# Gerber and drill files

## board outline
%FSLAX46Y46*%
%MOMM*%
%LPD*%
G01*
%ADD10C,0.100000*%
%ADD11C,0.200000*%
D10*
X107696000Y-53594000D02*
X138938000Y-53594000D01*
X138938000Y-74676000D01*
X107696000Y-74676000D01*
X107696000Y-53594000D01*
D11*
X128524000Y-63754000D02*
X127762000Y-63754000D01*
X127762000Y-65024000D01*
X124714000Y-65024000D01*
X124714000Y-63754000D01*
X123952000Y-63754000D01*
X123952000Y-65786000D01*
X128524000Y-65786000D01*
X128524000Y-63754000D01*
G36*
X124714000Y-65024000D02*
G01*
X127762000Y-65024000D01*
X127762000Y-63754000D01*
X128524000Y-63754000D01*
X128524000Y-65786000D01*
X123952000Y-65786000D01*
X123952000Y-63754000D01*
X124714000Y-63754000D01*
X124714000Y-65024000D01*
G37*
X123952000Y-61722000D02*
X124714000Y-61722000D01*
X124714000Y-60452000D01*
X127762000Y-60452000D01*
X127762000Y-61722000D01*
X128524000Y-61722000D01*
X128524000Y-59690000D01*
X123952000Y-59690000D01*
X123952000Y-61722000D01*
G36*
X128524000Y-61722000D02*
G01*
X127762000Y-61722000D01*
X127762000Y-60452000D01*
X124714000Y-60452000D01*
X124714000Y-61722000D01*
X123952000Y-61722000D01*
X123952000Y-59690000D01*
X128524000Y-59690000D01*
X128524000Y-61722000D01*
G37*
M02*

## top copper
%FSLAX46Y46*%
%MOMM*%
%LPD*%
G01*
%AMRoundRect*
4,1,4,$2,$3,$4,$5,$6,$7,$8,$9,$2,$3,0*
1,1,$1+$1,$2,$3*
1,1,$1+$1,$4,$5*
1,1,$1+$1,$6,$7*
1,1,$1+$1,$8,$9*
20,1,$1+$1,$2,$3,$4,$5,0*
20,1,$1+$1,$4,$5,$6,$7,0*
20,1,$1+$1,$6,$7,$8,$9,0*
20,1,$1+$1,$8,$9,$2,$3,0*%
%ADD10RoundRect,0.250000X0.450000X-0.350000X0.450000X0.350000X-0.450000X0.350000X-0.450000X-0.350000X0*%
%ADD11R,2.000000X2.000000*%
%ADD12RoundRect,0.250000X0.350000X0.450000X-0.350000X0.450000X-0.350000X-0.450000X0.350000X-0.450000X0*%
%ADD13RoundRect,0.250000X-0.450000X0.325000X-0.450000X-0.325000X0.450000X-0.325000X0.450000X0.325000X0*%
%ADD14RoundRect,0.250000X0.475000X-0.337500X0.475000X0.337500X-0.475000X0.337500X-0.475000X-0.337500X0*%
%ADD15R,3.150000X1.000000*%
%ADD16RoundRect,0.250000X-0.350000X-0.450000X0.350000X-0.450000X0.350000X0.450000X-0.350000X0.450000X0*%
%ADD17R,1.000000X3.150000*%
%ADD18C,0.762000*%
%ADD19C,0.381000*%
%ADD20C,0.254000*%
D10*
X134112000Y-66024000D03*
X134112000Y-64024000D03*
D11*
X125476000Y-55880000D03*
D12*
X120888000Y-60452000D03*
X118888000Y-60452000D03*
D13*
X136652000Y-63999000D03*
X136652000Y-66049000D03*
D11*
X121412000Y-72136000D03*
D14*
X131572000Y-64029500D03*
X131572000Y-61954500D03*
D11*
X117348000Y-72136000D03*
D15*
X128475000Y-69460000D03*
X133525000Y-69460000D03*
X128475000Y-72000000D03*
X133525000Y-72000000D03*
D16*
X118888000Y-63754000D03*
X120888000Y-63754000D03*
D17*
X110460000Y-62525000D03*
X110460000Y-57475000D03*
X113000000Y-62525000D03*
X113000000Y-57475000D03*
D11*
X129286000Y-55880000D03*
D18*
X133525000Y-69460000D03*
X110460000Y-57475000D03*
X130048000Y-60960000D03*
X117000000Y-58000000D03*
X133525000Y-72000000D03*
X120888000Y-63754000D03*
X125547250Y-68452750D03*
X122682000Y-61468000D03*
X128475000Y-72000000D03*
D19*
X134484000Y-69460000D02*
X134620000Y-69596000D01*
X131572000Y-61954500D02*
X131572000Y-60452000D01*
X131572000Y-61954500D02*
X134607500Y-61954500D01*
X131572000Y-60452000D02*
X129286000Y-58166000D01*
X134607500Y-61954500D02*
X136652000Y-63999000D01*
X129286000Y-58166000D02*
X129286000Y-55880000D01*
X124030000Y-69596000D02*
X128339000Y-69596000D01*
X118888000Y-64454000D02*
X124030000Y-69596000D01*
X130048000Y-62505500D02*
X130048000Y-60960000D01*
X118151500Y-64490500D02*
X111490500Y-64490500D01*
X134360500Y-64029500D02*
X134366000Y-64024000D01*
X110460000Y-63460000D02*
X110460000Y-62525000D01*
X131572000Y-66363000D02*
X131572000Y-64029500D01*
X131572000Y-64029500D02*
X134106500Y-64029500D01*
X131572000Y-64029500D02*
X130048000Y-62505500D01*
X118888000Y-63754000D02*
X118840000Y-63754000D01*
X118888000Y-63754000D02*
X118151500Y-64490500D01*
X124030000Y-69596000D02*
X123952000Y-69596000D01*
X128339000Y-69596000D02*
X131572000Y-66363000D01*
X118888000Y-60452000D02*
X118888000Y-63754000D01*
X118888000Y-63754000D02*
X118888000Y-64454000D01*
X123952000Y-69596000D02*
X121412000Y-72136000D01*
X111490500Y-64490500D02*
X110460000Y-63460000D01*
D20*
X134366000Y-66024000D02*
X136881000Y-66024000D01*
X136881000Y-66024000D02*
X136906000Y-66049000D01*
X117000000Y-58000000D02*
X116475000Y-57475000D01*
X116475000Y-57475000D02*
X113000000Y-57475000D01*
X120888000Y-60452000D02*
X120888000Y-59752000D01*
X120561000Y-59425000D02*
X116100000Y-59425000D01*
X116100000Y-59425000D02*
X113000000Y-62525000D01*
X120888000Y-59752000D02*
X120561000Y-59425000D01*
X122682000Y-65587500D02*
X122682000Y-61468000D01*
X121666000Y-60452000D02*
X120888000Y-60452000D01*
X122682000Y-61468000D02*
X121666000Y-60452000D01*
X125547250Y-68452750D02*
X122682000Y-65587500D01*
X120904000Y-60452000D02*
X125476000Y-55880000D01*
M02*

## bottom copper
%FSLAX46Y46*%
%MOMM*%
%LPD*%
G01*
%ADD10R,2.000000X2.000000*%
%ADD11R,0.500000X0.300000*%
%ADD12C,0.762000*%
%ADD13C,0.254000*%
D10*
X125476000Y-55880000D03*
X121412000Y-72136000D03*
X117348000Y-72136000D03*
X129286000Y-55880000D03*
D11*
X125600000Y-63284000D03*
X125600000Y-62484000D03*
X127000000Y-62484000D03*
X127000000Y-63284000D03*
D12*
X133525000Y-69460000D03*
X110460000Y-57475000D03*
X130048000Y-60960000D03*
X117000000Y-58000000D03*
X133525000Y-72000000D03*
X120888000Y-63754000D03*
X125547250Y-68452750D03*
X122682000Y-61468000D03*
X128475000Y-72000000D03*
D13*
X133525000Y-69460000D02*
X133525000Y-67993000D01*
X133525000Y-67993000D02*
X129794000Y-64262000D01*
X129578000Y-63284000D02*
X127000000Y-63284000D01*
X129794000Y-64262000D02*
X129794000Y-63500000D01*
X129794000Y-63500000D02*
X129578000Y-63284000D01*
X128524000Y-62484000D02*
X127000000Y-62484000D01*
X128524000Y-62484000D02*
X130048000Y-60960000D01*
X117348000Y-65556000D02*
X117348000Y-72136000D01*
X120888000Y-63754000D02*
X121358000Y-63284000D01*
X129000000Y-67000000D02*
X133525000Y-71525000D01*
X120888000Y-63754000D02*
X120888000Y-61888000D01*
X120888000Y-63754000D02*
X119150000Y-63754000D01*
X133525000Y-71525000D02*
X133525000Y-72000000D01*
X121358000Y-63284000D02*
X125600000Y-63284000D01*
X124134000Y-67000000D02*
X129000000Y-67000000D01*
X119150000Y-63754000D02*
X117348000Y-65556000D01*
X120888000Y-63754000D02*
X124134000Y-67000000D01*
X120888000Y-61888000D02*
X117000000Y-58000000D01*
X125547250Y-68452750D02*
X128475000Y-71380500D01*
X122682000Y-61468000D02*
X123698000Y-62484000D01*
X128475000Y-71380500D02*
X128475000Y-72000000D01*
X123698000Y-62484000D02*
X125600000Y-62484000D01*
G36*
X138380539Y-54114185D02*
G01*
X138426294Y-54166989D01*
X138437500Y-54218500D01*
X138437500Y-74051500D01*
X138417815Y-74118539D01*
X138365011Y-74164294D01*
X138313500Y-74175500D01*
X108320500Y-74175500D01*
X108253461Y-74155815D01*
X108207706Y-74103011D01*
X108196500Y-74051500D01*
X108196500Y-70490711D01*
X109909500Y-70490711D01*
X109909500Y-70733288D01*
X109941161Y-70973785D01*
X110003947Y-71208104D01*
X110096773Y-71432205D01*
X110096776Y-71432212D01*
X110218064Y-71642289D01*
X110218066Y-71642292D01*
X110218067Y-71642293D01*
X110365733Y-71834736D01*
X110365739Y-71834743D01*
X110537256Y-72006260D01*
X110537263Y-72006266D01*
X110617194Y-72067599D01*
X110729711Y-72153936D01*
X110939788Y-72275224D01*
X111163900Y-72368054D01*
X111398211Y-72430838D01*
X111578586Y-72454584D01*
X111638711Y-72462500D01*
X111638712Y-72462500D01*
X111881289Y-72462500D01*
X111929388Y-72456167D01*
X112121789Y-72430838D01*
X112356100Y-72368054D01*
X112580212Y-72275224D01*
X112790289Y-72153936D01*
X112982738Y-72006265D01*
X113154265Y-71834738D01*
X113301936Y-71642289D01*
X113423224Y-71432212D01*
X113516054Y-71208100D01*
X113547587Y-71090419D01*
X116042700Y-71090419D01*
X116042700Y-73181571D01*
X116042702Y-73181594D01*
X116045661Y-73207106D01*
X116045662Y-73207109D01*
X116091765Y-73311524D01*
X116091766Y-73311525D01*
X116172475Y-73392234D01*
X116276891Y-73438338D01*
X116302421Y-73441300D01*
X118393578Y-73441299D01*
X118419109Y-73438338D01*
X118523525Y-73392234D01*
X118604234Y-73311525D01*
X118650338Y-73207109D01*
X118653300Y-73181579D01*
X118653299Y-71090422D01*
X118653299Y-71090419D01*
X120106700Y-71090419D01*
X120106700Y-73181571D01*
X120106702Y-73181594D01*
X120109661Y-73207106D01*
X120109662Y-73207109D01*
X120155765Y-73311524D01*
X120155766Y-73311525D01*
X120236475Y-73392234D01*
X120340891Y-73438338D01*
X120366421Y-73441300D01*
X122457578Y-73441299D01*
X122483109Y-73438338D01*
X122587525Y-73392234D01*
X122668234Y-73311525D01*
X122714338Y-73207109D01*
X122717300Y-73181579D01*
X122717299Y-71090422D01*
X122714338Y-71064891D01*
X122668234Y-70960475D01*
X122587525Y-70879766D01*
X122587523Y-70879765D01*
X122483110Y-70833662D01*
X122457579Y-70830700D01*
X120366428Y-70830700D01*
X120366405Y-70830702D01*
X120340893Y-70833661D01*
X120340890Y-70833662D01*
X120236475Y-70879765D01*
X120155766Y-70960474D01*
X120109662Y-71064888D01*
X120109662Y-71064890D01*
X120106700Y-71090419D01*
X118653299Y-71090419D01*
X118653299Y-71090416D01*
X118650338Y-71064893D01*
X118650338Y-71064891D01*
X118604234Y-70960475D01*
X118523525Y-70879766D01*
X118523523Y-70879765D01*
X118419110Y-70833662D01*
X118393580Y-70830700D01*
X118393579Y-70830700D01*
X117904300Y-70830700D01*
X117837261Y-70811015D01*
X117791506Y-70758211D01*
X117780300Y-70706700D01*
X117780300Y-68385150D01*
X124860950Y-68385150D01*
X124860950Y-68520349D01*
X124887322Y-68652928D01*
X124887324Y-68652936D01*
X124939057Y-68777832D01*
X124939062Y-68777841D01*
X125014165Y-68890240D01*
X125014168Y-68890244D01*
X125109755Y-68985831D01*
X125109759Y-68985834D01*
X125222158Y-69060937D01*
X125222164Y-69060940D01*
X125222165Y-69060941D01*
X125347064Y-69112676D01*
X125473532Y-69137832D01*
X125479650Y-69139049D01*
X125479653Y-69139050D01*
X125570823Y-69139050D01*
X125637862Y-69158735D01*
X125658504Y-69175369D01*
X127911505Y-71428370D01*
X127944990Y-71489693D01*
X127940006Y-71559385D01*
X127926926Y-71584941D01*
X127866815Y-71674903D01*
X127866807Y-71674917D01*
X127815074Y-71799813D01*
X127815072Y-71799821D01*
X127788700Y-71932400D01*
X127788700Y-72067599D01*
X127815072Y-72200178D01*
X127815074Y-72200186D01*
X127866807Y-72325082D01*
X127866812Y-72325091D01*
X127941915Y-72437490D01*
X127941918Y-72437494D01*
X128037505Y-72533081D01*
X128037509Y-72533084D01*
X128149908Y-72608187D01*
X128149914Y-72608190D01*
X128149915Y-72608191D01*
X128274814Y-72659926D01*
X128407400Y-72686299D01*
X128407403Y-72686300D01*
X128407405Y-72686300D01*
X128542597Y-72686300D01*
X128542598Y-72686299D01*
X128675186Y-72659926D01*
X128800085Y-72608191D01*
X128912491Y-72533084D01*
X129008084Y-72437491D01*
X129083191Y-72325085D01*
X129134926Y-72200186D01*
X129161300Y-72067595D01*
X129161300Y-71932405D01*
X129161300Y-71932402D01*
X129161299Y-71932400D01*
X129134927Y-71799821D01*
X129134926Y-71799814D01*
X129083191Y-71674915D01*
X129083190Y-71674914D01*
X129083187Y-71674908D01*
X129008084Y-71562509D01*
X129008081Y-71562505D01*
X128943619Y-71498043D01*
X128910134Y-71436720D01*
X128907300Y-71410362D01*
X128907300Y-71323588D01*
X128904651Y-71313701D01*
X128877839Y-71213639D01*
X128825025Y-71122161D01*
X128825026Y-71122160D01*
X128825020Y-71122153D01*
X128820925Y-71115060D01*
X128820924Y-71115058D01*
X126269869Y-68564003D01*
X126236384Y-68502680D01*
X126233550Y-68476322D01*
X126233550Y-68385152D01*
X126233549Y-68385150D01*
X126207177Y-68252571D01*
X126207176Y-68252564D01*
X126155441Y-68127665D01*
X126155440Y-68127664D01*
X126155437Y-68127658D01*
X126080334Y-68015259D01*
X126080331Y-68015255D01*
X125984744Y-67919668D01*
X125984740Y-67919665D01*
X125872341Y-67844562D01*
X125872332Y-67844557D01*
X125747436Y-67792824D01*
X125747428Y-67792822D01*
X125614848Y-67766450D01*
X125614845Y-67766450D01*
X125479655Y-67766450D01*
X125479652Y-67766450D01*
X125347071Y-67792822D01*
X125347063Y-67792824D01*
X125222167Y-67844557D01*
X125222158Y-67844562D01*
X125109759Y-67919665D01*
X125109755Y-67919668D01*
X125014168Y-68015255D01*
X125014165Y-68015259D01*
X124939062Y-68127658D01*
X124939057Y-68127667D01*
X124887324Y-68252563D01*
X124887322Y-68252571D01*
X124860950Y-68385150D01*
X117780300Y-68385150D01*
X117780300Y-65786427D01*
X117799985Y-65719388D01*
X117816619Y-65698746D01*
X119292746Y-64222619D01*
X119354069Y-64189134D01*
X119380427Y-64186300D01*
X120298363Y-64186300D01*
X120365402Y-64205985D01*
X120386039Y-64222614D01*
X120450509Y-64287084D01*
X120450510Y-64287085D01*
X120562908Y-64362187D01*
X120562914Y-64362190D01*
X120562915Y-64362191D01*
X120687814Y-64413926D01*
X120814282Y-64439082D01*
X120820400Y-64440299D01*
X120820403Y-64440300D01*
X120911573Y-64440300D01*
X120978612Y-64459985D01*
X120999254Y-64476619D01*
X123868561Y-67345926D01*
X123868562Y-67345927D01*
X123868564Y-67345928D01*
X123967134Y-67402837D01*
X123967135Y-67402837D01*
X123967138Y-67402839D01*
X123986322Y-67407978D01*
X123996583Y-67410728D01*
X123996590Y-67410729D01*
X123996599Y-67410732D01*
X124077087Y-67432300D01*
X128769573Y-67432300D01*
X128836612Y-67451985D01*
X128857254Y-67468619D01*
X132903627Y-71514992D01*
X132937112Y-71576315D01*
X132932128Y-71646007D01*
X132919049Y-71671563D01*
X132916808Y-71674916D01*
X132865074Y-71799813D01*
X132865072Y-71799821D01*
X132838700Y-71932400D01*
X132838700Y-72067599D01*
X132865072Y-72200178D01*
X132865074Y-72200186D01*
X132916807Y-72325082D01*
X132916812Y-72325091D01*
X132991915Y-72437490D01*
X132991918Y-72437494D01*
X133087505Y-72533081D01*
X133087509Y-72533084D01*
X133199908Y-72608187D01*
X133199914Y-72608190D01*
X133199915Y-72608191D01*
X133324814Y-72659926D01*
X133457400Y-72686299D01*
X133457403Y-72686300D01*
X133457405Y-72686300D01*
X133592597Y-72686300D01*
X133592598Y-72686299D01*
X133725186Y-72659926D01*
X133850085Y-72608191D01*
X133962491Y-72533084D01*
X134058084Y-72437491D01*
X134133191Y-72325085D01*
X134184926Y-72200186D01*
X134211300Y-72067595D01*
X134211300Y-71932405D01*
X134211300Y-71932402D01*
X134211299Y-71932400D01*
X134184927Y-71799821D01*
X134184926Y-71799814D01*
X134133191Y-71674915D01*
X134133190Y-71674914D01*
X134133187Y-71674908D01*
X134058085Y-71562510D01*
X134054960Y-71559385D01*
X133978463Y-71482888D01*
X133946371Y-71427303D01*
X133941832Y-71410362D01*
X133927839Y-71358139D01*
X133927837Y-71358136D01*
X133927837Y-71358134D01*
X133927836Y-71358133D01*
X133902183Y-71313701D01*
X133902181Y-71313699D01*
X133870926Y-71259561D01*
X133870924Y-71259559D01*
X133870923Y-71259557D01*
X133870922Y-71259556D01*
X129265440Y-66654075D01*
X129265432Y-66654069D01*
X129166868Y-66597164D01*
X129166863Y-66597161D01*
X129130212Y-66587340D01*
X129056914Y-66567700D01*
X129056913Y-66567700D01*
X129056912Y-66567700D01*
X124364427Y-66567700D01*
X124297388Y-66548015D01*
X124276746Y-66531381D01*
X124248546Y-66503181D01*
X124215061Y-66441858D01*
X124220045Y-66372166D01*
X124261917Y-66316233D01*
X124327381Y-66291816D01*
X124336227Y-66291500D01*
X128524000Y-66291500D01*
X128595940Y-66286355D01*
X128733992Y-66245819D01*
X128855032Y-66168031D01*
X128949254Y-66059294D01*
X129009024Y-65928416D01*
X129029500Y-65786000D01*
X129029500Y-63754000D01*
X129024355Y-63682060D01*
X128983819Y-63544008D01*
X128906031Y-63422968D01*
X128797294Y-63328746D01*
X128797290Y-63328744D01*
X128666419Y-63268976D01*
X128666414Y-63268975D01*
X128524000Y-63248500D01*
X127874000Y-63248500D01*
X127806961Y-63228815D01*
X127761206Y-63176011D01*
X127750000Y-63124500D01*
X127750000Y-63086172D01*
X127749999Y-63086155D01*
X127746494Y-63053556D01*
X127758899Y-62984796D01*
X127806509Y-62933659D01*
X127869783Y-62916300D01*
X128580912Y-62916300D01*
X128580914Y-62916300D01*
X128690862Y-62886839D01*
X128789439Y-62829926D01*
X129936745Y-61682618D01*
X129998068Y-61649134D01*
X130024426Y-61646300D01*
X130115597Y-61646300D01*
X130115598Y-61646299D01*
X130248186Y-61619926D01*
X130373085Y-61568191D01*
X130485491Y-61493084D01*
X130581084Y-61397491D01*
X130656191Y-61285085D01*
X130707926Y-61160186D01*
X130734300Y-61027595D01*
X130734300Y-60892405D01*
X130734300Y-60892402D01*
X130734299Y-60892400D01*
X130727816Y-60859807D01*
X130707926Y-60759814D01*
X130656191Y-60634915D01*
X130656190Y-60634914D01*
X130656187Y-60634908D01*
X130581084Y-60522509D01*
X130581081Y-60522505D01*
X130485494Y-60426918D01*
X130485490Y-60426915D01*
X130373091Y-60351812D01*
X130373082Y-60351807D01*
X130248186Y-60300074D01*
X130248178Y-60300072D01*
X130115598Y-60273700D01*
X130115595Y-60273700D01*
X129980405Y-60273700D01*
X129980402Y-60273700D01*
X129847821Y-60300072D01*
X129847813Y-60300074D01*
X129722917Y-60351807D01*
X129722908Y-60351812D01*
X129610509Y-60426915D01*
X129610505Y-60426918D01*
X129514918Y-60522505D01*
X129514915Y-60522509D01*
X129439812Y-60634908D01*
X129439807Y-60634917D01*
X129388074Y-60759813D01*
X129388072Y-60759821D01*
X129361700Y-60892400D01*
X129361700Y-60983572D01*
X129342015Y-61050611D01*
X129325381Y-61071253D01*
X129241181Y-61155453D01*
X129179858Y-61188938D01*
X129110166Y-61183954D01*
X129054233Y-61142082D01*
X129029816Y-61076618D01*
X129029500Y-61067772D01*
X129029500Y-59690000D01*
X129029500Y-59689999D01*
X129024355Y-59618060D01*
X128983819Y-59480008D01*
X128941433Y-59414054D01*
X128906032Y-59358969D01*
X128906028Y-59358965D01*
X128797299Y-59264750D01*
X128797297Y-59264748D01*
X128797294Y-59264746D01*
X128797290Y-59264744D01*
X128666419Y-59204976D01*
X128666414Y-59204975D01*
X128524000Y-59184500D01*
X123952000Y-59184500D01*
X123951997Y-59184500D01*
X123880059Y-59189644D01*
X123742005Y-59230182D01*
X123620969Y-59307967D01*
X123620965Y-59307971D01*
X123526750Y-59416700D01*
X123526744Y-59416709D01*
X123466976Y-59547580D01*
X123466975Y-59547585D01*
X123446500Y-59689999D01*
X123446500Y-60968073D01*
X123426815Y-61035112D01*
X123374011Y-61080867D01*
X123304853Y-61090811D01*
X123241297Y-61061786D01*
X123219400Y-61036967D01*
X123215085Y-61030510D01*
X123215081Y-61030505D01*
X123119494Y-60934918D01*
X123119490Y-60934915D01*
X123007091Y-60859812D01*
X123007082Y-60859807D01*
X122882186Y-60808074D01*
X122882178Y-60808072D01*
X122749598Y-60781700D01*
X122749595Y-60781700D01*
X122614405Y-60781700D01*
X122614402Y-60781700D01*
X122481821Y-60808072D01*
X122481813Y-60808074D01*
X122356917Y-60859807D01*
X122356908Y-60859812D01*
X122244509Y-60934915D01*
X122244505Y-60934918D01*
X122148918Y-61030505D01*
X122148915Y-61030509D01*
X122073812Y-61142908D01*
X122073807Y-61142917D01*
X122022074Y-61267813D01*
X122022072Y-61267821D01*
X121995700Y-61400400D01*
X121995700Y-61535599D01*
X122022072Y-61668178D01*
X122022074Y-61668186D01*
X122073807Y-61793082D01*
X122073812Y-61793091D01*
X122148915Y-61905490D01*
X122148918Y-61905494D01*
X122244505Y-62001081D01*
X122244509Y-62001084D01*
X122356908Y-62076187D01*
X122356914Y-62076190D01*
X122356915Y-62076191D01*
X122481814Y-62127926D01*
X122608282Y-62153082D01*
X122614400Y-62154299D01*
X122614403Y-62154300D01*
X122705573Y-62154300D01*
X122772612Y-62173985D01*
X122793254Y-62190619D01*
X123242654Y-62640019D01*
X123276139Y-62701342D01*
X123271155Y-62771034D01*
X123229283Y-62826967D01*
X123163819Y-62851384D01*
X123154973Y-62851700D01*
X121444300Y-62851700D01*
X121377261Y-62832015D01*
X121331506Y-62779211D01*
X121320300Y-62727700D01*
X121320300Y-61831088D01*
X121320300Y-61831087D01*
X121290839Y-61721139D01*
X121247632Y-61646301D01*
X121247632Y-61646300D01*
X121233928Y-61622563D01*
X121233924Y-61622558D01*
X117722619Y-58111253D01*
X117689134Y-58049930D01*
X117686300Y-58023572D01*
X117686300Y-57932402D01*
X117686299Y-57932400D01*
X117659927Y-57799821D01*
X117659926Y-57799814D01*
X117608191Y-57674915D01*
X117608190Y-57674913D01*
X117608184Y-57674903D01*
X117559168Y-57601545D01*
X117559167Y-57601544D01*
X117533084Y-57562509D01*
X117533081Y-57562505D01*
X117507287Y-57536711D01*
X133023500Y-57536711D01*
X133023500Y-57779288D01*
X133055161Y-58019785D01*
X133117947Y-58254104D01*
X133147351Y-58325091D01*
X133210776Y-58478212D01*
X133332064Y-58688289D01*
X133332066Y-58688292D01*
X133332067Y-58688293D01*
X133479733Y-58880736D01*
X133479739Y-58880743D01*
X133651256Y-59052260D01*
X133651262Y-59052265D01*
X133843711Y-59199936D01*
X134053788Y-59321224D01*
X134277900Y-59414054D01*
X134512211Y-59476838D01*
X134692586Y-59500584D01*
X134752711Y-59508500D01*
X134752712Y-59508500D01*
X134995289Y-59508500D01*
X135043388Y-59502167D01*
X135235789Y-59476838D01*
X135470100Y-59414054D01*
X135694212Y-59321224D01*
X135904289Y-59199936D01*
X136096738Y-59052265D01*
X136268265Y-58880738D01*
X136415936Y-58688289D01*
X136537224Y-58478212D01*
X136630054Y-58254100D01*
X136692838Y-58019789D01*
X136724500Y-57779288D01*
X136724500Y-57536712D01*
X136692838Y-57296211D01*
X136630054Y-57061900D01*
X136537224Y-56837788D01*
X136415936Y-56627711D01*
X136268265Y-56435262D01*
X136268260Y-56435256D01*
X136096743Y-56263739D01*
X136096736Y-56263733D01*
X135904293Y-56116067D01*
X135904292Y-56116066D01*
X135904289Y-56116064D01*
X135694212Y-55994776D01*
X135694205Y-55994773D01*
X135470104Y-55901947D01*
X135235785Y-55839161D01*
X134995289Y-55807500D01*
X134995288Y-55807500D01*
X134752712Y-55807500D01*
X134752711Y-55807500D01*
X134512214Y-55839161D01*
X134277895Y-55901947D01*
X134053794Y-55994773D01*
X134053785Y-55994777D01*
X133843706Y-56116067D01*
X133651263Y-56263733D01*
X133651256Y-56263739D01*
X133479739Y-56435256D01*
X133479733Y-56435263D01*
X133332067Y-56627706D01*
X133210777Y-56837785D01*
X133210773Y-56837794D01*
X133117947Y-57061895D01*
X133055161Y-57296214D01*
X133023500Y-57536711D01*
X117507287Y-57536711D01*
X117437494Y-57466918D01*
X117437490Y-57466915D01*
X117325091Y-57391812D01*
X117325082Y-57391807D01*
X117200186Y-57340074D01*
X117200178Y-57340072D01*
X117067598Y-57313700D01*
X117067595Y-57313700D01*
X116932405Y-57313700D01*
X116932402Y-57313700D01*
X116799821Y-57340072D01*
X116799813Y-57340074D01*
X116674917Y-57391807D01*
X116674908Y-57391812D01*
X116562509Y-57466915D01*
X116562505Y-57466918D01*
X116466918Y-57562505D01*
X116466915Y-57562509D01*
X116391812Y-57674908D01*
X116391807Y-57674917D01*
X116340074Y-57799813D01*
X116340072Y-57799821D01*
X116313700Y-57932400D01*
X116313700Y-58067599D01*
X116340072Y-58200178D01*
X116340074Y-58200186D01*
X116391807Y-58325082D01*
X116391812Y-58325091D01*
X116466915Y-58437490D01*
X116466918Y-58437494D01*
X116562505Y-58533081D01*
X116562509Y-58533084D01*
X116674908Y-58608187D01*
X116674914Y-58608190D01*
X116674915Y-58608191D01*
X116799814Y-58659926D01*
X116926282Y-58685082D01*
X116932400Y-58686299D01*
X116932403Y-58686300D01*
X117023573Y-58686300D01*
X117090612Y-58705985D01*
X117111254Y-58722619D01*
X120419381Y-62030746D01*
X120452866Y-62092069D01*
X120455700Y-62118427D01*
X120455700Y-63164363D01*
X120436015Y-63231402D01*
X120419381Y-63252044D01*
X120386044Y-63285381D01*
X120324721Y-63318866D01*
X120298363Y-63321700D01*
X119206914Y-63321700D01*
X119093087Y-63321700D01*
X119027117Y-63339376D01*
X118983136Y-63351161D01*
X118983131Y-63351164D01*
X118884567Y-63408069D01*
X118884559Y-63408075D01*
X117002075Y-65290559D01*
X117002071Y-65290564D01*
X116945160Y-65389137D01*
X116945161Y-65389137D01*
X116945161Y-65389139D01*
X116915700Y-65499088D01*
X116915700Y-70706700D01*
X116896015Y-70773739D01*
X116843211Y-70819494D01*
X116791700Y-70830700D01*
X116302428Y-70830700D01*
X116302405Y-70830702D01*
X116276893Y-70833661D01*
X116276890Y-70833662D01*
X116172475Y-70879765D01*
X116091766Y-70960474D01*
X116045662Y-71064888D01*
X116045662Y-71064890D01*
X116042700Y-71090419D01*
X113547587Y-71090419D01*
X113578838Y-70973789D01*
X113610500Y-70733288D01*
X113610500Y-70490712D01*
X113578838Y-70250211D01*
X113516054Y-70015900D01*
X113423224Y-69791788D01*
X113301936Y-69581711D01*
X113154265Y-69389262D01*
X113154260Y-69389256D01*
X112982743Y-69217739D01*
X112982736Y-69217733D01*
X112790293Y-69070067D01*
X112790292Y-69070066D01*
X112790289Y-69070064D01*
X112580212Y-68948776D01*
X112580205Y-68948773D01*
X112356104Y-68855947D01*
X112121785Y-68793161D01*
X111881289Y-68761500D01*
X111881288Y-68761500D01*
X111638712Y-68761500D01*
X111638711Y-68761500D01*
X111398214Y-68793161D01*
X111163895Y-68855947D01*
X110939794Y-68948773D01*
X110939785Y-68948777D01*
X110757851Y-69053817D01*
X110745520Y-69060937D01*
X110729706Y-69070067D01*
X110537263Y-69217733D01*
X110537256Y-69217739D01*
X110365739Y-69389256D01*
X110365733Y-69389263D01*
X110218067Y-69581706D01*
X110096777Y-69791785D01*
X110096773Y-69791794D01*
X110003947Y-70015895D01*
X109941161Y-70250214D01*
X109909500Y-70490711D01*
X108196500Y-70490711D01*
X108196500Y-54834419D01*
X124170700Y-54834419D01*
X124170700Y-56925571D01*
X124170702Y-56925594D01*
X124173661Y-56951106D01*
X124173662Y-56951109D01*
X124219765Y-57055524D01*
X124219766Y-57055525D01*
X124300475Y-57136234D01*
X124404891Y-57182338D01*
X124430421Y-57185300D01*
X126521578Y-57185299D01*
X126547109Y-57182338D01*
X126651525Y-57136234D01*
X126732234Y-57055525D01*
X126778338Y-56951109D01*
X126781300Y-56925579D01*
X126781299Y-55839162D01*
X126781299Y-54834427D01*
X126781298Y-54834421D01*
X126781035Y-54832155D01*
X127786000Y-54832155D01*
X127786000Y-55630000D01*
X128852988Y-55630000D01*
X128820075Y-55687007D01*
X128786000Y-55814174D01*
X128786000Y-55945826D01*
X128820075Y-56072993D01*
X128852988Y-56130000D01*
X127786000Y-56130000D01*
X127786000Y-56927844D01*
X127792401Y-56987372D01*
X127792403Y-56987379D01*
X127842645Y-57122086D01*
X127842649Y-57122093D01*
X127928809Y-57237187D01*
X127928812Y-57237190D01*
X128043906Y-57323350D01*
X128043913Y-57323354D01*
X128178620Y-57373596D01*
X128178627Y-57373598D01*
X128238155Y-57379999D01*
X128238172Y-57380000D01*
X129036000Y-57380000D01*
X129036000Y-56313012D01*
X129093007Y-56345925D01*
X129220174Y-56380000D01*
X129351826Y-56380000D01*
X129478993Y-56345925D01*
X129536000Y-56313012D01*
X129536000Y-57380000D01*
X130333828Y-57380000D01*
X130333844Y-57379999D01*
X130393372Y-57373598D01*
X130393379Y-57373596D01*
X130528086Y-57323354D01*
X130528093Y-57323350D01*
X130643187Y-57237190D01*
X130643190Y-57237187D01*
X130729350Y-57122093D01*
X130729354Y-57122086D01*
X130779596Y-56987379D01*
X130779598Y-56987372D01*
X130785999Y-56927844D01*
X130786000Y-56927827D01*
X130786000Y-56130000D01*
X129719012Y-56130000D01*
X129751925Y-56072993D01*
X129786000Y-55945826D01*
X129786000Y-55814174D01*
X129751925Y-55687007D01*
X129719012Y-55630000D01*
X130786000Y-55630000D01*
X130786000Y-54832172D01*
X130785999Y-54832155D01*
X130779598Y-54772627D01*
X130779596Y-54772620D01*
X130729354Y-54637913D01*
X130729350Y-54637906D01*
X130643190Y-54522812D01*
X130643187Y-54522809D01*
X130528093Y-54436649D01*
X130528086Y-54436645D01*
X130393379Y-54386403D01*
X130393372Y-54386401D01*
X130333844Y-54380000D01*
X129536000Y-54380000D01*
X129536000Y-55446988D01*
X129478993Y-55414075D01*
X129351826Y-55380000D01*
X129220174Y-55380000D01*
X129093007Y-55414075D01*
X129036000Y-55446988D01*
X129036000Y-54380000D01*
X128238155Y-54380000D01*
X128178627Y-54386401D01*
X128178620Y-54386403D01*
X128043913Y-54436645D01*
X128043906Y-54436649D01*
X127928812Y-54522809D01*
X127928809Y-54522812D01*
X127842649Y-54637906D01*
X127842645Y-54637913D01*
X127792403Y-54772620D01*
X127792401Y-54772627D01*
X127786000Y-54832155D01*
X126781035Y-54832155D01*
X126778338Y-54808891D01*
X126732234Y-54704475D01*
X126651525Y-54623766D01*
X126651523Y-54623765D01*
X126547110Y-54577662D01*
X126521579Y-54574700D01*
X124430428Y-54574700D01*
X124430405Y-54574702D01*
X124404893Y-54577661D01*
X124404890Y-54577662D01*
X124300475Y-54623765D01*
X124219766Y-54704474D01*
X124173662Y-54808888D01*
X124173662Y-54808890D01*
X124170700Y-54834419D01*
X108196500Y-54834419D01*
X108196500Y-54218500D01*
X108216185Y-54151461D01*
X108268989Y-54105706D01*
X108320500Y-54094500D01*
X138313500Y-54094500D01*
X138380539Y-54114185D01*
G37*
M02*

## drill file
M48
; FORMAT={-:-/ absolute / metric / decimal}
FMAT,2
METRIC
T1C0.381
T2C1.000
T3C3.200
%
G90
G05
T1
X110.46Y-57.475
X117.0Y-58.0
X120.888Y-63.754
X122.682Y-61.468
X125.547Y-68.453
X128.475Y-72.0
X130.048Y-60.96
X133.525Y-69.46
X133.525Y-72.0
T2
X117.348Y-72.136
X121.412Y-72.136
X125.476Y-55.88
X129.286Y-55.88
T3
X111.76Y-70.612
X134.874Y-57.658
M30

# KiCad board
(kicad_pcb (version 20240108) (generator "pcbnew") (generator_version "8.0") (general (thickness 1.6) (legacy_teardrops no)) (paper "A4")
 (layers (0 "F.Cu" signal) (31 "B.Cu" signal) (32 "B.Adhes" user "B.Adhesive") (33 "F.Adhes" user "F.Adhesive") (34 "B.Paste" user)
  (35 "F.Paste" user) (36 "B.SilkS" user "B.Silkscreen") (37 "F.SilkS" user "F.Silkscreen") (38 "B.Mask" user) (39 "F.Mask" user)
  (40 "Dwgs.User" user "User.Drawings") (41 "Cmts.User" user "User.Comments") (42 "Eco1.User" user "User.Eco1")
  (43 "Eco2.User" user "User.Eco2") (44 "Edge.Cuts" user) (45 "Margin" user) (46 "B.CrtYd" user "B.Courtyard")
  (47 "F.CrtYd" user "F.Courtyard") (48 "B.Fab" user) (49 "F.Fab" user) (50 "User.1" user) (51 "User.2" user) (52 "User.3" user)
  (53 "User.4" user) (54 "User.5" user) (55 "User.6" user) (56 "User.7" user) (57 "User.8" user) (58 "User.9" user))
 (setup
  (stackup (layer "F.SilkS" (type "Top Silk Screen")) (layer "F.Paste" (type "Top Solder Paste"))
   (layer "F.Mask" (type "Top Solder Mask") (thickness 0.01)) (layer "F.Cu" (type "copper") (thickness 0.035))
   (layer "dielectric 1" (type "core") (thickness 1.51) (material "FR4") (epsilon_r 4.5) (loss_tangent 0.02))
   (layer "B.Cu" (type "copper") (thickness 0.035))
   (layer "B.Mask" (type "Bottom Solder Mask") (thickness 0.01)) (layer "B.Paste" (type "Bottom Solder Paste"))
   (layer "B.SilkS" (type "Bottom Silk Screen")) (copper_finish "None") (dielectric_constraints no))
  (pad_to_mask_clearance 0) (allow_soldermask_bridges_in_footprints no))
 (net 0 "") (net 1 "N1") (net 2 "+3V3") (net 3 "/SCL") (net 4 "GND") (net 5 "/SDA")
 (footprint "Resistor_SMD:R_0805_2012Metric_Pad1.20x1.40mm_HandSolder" (layer "F.Cu") (at 134.112 65.024 90)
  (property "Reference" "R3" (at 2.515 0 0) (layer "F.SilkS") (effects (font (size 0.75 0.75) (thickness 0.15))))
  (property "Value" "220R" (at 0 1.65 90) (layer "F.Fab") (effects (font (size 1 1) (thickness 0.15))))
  (pad "1" smd roundrect (at -1 0 90) (size 1.2 1.4) (layers "F.Cu" "F.Paste" "F.Mask") (roundrect_rratio 0.208333) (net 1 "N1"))
  (pad "2" smd roundrect (at 1 0 90) (size 1.2 1.4) (layers "F.Cu" "F.Paste" "F.Mask") (roundrect_rratio 0.208333) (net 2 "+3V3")))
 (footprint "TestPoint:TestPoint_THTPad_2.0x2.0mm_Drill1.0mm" (layer "F.Cu") (at 125.476 55.88)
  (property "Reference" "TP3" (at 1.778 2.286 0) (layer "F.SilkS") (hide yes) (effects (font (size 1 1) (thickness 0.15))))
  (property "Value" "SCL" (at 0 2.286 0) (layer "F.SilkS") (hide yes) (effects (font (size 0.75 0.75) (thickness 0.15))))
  (pad "1" thru_hole rect (at 0 0) (size 2 2) (drill 1) (layers "*.Cu" "*.Mask") (remove_unused_layers no) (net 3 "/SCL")))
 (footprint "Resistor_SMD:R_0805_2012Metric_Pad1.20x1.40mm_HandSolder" (layer "F.Cu") (at 119.888 60.452 180)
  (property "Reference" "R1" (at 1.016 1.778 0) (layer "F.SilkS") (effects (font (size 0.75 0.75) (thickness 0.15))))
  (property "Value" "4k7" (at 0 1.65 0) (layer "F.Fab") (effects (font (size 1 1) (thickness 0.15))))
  (pad "1" smd roundrect (at -1 0 180) (size 1.2 1.4) (layers "F.Cu" "F.Paste" "F.Mask") (roundrect_rratio 0.208333) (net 3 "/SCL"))
  (pad "2" smd roundrect (at 1 0 180) (size 1.2 1.4) (layers "F.Cu" "F.Paste" "F.Mask") (roundrect_rratio 0.208333) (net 2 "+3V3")))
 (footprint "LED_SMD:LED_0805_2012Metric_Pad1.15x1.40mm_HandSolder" (layer "F.Cu") (at 136.652 65.024 -90)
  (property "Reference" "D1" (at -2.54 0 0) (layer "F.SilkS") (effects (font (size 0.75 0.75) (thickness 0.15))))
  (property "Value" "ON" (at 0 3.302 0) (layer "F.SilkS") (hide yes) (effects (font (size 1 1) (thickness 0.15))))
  (pad "1" smd roundrect (at -1.025 0 270) (size 1.15 1.4) (layers "F.Cu" "F.Paste" "F.Mask") (roundrect_rratio 0.217391) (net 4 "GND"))
  (pad "2" smd roundrect (at 1.025 0 270) (size 1.15 1.4) (layers "F.Cu" "F.Paste" "F.Mask") (roundrect_rratio 0.217391) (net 1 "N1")))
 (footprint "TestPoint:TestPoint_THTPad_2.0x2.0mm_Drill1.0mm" (layer "F.Cu") (at 121.412 72.136)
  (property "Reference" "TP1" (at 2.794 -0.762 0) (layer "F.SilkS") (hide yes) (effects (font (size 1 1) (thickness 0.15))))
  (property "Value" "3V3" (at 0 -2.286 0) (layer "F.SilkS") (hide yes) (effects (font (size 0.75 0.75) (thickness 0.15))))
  (pad "1" thru_hole rect (at 0 0) (size 2 2) (drill 1) (layers "*.Cu" "*.Mask") (remove_unused_layers no) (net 2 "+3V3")))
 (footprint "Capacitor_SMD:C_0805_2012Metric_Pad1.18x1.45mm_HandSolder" (layer "F.Cu") (at 131.572 62.992 90)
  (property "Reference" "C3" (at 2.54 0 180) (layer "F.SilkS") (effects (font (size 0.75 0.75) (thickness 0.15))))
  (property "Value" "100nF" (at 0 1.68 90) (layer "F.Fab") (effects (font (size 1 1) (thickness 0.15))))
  (pad "1" smd roundrect (at -1.0375 0 90) (size 1.175 1.45) (layers "F.Cu" "F.Paste" "F.Mask") (roundrect_rratio 0.212766) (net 2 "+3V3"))
  (pad "2" smd roundrect (at 1.0375 0 90) (size 1.175 1.45) (layers "F.Cu" "F.Paste" "F.Mask") (roundrect_rratio 0.212766) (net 4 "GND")))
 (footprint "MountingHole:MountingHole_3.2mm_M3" (layer "F.Cu") (at 134.874 57.658)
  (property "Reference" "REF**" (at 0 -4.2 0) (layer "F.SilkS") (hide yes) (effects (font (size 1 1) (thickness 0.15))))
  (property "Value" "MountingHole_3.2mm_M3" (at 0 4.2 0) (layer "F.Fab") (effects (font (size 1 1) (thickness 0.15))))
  (pad "" np_thru_hole circle (at 0 0) (size 3.2 3.2) (drill 3.2) (layers "*.Cu" "*.Mask")))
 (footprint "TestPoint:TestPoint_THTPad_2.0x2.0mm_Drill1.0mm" (layer "F.Cu") (at 117.348 72.136)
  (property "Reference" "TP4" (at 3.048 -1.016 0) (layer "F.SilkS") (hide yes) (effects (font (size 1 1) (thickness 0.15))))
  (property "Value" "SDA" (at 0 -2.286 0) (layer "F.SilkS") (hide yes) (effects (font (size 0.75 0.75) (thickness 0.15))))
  (pad "1" thru_hole rect (at 0 0) (size 2 2) (drill 1) (layers "*.Cu" "*.Mask") (remove_unused_layers no) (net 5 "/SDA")))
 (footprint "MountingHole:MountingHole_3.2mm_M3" (layer "F.Cu") (at 111.76 70.612)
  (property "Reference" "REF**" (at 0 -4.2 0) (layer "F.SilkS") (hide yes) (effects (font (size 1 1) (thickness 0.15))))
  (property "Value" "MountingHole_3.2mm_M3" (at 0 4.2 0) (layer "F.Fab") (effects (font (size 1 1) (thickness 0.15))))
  (pad "" np_thru_hole circle (at 0 0) (size 3.2 3.2) (drill 3.2) (layers "*.Cu" "*.Mask")))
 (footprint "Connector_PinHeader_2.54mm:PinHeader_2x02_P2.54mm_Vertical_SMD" (layer "F.Cu") (at 131 70.73)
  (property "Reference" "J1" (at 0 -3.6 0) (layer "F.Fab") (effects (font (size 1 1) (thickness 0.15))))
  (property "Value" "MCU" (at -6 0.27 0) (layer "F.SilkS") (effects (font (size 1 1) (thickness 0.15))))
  (pad "1" smd rect (at -2.525 -1.27) (size 3.15 1) (layers "F.Cu" "F.Paste" "F.Mask") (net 2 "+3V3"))
  (pad "2" smd rect (at 2.525 -1.27) (size 3.15 1) (layers "F.Cu" "F.Paste" "F.Mask") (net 4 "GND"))
  (pad "3" smd rect (at -2.525 1.27) (size 3.15 1) (layers "F.Cu" "F.Paste" "F.Mask") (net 3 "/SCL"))
  (pad "4" smd rect (at 2.525 1.27) (size 3.15 1) (layers "F.Cu" "F.Paste" "F.Mask") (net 5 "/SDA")))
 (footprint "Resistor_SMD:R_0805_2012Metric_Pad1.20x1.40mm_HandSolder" (layer "F.Cu") (at 119.888 63.754)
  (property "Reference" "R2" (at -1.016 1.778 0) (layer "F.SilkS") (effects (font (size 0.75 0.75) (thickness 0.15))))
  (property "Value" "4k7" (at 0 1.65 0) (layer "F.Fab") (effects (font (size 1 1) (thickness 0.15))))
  (pad "1" smd roundrect (at -1 0) (size 1.2 1.4) (layers "F.Cu" "F.Paste" "F.Mask") (roundrect_rratio 0.208333) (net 2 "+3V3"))
  (pad "2" smd roundrect (at 1 0) (size 1.2 1.4) (layers "F.Cu" "F.Paste" "F.Mask") (roundrect_rratio 0.208333) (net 5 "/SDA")))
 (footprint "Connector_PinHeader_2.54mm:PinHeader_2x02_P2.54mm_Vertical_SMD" (layer "F.Cu") (at 111.73 60 90)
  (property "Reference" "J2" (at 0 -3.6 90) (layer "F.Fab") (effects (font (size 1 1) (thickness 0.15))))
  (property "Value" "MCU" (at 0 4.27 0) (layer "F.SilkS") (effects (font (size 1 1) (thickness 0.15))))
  (pad "1" smd rect (at -2.525 -1.27 90) (size 3.15 1) (layers "F.Cu" "F.Paste" "F.Mask") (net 2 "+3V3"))
  (pad "2" smd rect (at 2.525 -1.27 90) (size 3.15 1) (layers "F.Cu" "F.Paste" "F.Mask") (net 4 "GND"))
  (pad "3" smd rect (at -2.525 1.27 90) (size 3.15 1) (layers "F.Cu" "F.Paste" "F.Mask") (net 3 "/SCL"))
  (pad "4" smd rect (at 2.525 1.27 90) (size 3.15 1) (layers "F.Cu" "F.Paste" "F.Mask") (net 5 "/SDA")))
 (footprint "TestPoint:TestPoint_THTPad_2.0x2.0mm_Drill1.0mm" (layer "F.Cu") (at 129.286 55.88)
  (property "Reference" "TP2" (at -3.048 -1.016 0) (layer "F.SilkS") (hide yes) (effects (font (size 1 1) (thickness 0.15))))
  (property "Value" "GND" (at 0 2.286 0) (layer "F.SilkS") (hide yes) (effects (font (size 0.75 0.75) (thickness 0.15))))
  (pad "1" thru_hole rect (at 0 0) (size 2 2) (drill 1) (layers "*.Cu" "*.Mask") (remove_unused_layers no) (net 4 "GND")))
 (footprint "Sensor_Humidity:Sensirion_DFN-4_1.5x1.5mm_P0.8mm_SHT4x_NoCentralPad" (layer "B.Cu") (at 126.3 62.884)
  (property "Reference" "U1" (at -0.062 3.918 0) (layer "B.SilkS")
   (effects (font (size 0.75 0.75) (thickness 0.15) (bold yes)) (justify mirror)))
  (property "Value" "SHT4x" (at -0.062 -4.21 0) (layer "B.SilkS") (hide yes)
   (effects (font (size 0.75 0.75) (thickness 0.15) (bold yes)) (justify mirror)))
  (pad "1" smd rect (at -0.7 0.4) (size 0.5 0.3) (layers "B.Cu" "B.Paste" "B.Mask") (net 5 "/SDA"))
  (pad "2" smd rect (at -0.7 -0.4) (size 0.5 0.3) (layers "B.Cu" "B.Paste" "B.Mask") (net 3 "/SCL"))
  (pad "3" smd rect (at 0.7 -0.4) (size 0.5 0.3) (layers "B.Cu" "B.Paste" "B.Mask") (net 2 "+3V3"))
  (pad "4" smd rect (at 0.7 0.4) (size 0.5 0.3) (layers "B.Cu" "B.Paste" "B.Mask") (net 4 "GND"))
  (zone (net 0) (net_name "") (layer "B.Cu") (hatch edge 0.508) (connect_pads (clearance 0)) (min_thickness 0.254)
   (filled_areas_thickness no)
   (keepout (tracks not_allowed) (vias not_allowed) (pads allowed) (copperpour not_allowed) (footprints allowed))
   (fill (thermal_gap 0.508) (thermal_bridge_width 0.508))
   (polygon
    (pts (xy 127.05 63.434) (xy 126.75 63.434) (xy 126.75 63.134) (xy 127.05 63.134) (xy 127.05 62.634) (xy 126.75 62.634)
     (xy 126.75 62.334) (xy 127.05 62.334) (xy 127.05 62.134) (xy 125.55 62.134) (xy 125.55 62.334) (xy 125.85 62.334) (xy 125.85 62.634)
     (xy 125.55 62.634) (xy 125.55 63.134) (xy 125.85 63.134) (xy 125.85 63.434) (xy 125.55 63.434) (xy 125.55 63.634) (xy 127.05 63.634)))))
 (gr_rect (start 107.696 53.594) (end 138.938 74.676) (stroke (width 0.1) (type default)) (fill none) (layer "Edge.Cuts"))
 (gr_poly
  (pts (xy 128.524 63.754) (xy 127.762 63.754) (xy 127.762 65.024) (xy 124.714 65.024) (xy 124.714 63.754) (xy 123.952 63.754)
   (xy 123.952 65.786) (xy 128.524 65.786))
  (stroke (width 0.2) (type solid)) (fill solid) (layer "Edge.Cuts"))
 (gr_poly
  (pts (xy 123.952 61.722) (xy 124.714 61.722) (xy 124.714 60.452) (xy 127.762 60.452) (xy 127.762 61.722) (xy 128.524 61.722)
   (xy 128.524 59.69) (xy 123.952 59.69))
  (stroke (width 0.2) (type solid)) (fill solid) (layer "Edge.Cuts"))
 (segment (start 134.484 69.46) (end 134.62 69.596) (width 0.381) (layer "F.Cu") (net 4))
 (segment (start 131.572 61.9545) (end 131.572 60.452) (width 0.381) (layer "F.Cu") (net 4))
 (segment (start 131.572 61.9545) (end 134.6075 61.9545) (width 0.381) (layer "F.Cu") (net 4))
 (segment (start 131.572 60.452) (end 129.286 58.166) (width 0.381) (layer "F.Cu") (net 4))
 (segment (start 134.6075 61.9545) (end 136.652 63.999) (width 0.381) (layer "F.Cu") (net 4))
 (segment (start 129.286 58.166) (end 129.286 55.88) (width 0.381) (layer "F.Cu") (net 4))
 (via (at 133.525 69.46) (size 0.762) (drill 0.381) (layers "F.Cu" "B.Cu") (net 4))
 (via (at 110.46 57.475) (size 0.762) (drill 0.381) (layers "F.Cu" "B.Cu") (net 4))
 (segment (start 133.525 69.46) (end 133.525 67.993) (width 0.254) (layer "B.Cu") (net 4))
 (segment (start 133.525 67.993) (end 129.794 64.262) (width 0.254) (layer "B.Cu") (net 4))
 (segment (start 129.578 63.284) (end 127 63.284) (width 0.254) (layer "B.Cu") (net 4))
 (segment (start 129.794 64.262) (end 129.794 63.5) (width 0.254) (layer "B.Cu") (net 4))
 (segment (start 129.794 63.5) (end 129.578 63.284) (width 0.254) (layer "B.Cu") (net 4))
 (segment (start 124.03 69.596) (end 128.339 69.596) (width 0.381) (layer "F.Cu") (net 2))
 (segment (start 118.888 64.454) (end 124.03 69.596) (width 0.381) (layer "F.Cu") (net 2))
 (segment (start 130.048 62.5055) (end 130.048 60.96) (width 0.381) (layer "F.Cu") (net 2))
 (segment (start 118.1515 64.4905) (end 111.4905 64.4905) (width 0.381) (layer "F.Cu") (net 2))
 (segment (start 134.3605 64.0295) (end 134.366 64.024) (width 0.381) (layer "F.Cu") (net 2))
 (segment (start 110.46 63.46) (end 110.46 62.525) (width 0.381) (layer "F.Cu") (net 2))
 (segment (start 131.572 66.363) (end 131.572 64.0295) (width 0.381) (layer "F.Cu") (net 2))
 (segment (start 131.572 64.0295) (end 134.1065 64.0295) (width 0.381) (layer "F.Cu") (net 2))
 (segment (start 131.572 64.0295) (end 130.048 62.5055) (width 0.381) (layer "F.Cu") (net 2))
 (segment (start 118.888 63.754) (end 118.84 63.754) (width 0.381) (layer "F.Cu") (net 2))
 (segment (start 118.888 63.754) (end 118.1515 64.4905) (width 0.381) (layer "F.Cu") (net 2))
 (segment (start 124.03 69.596) (end 123.952 69.596) (width 0.381) (layer "F.Cu") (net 2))
 (segment (start 128.339 69.596) (end 131.572 66.363) (width 0.381) (layer "F.Cu") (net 2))
 (segment (start 118.888 60.452) (end 118.888 63.754) (width 0.381) (layer "F.Cu") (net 2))
 (segment (start 118.888 63.754) (end 118.888 64.454) (width 0.381) (layer "F.Cu") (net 2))
 (segment (start 123.952 69.596) (end 121.412 72.136) (width 0.381) (layer "F.Cu") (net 2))
 (segment (start 111.4905 64.4905) (end 110.46 63.46) (width 0.381) (layer "F.Cu") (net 2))
 (via (at 130.048 60.96) (size 0.762) (drill 0.381) (layers "F.Cu" "B.Cu") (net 2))
 (segment (start 128.524 62.484) (end 127 62.484) (width 0.254) (layer "B.Cu") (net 2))
 (segment (start 128.524 62.484) (end 130.048 60.96) (width 0.254) (layer "B.Cu") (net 2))
 (segment (start 134.366 66.024) (end 136.881 66.024) (width 0.254) (layer "F.Cu") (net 1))
 (segment (start 136.881 66.024) (end 136.906 66.049) (width 0.254) (layer "F.Cu") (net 1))
 (segment (start 117 58) (end 116.475 57.475) (width 0.254) (layer "F.Cu") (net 5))
 (segment (start 116.475 57.475) (end 113 57.475) (width 0.254) (layer "F.Cu") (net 5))
 (via (at 117 58) (size 0.762) (drill 0.381) (layers "F.Cu" "B.Cu") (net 5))
 (via (at 133.525 72) (size 0.762) (drill 0.381) (layers "F.Cu" "B.Cu") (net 5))
 (via (at 120.888 63.754) (size 0.762) (drill 0.381) (layers "F.Cu" "B.Cu") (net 5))
 (segment (start 117.348 65.556) (end 117.348 72.136) (width 0.254) (layer "B.Cu") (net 5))
 (segment (start 120.888 63.754) (end 121.358 63.284) (width 0.254) (layer "B.Cu") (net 5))
 (segment (start 129 67) (end 133.525 71.525) (width 0.254) (layer "B.Cu") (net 5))
 (segment (start 120.888 63.754) (end 120.888 61.888) (width 0.254) (layer "B.Cu") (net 5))
 (segment (start 120.888 63.754) (end 119.15 63.754) (width 0.254) (layer "B.Cu") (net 5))
 (segment (start 133.525 71.525) (end 133.525 72) (width 0.254) (layer "B.Cu") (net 5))
 (segment (start 121.358 63.284) (end 125.6 63.284) (width 0.254) (layer "B.Cu") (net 5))
 (segment (start 124.134 67) (end 129 67) (width 0.254) (layer "B.Cu") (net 5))
 (segment (start 119.15 63.754) (end 117.348 65.556) (width 0.254) (layer "B.Cu") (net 5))
 (segment (start 120.888 63.754) (end 124.134 67) (width 0.254) (layer "B.Cu") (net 5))
 (segment (start 120.888 61.888) (end 117 58) (width 0.254) (layer "B.Cu") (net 5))
 (segment (start 120.888 60.452) (end 120.888 59.752) (width 0.254) (layer "F.Cu") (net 3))
 (segment (start 120.561 59.425) (end 116.1 59.425) (width 0.254) (layer "F.Cu") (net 3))
 (segment (start 116.1 59.425) (end 113 62.525) (width 0.254) (layer "F.Cu") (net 3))
 (segment (start 120.888 59.752) (end 120.561 59.425) (width 0.254) (layer "F.Cu") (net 3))
 (segment (start 122.682 65.5875) (end 122.682 61.468) (width 0.254) (layer "F.Cu") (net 3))
 (segment (start 121.666 60.452) (end 120.888 60.452) (width 0.254) (layer "F.Cu") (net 3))
 (segment (start 122.682 61.468) (end 121.666 60.452) (width 0.254) (layer "F.Cu") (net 3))
 (segment (start 125.54725 68.45275) (end 122.682 65.5875) (width 0.254) (layer "F.Cu") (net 3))
 (segment (start 120.904 60.452) (end 125.476 55.88) (width 0.254) (layer "F.Cu") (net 3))
 (via (at 125.54725 68.45275) (size 0.762) (drill 0.381) (layers "F.Cu" "B.Cu") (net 3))
 (via (at 122.682 61.468) (size 0.762) (drill 0.381) (layers "F.Cu" "B.Cu") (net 3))
 (via (at 128.475 72) (size 0.762) (drill 0.381) (layers "F.Cu" "B.Cu") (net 3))
 (segment (start 125.54725 68.45275) (end 128.475 71.3805) (width 0.254) (layer "B.Cu") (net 3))
 (segment (start 122.682 61.468) (end 123.698 62.484) (width 0.254) (layer "B.Cu") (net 3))
 (segment (start 128.475 71.3805) (end 128.475 72) (width 0.254) (layer "B.Cu") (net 3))
 (segment (start 123.698 62.484) (end 125.6 62.484) (width 0.254) (layer "B.Cu") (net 3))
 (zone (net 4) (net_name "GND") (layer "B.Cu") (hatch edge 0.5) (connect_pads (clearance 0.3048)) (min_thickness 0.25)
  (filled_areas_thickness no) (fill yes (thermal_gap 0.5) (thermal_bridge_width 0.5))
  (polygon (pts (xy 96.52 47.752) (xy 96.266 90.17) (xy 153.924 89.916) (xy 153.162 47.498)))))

